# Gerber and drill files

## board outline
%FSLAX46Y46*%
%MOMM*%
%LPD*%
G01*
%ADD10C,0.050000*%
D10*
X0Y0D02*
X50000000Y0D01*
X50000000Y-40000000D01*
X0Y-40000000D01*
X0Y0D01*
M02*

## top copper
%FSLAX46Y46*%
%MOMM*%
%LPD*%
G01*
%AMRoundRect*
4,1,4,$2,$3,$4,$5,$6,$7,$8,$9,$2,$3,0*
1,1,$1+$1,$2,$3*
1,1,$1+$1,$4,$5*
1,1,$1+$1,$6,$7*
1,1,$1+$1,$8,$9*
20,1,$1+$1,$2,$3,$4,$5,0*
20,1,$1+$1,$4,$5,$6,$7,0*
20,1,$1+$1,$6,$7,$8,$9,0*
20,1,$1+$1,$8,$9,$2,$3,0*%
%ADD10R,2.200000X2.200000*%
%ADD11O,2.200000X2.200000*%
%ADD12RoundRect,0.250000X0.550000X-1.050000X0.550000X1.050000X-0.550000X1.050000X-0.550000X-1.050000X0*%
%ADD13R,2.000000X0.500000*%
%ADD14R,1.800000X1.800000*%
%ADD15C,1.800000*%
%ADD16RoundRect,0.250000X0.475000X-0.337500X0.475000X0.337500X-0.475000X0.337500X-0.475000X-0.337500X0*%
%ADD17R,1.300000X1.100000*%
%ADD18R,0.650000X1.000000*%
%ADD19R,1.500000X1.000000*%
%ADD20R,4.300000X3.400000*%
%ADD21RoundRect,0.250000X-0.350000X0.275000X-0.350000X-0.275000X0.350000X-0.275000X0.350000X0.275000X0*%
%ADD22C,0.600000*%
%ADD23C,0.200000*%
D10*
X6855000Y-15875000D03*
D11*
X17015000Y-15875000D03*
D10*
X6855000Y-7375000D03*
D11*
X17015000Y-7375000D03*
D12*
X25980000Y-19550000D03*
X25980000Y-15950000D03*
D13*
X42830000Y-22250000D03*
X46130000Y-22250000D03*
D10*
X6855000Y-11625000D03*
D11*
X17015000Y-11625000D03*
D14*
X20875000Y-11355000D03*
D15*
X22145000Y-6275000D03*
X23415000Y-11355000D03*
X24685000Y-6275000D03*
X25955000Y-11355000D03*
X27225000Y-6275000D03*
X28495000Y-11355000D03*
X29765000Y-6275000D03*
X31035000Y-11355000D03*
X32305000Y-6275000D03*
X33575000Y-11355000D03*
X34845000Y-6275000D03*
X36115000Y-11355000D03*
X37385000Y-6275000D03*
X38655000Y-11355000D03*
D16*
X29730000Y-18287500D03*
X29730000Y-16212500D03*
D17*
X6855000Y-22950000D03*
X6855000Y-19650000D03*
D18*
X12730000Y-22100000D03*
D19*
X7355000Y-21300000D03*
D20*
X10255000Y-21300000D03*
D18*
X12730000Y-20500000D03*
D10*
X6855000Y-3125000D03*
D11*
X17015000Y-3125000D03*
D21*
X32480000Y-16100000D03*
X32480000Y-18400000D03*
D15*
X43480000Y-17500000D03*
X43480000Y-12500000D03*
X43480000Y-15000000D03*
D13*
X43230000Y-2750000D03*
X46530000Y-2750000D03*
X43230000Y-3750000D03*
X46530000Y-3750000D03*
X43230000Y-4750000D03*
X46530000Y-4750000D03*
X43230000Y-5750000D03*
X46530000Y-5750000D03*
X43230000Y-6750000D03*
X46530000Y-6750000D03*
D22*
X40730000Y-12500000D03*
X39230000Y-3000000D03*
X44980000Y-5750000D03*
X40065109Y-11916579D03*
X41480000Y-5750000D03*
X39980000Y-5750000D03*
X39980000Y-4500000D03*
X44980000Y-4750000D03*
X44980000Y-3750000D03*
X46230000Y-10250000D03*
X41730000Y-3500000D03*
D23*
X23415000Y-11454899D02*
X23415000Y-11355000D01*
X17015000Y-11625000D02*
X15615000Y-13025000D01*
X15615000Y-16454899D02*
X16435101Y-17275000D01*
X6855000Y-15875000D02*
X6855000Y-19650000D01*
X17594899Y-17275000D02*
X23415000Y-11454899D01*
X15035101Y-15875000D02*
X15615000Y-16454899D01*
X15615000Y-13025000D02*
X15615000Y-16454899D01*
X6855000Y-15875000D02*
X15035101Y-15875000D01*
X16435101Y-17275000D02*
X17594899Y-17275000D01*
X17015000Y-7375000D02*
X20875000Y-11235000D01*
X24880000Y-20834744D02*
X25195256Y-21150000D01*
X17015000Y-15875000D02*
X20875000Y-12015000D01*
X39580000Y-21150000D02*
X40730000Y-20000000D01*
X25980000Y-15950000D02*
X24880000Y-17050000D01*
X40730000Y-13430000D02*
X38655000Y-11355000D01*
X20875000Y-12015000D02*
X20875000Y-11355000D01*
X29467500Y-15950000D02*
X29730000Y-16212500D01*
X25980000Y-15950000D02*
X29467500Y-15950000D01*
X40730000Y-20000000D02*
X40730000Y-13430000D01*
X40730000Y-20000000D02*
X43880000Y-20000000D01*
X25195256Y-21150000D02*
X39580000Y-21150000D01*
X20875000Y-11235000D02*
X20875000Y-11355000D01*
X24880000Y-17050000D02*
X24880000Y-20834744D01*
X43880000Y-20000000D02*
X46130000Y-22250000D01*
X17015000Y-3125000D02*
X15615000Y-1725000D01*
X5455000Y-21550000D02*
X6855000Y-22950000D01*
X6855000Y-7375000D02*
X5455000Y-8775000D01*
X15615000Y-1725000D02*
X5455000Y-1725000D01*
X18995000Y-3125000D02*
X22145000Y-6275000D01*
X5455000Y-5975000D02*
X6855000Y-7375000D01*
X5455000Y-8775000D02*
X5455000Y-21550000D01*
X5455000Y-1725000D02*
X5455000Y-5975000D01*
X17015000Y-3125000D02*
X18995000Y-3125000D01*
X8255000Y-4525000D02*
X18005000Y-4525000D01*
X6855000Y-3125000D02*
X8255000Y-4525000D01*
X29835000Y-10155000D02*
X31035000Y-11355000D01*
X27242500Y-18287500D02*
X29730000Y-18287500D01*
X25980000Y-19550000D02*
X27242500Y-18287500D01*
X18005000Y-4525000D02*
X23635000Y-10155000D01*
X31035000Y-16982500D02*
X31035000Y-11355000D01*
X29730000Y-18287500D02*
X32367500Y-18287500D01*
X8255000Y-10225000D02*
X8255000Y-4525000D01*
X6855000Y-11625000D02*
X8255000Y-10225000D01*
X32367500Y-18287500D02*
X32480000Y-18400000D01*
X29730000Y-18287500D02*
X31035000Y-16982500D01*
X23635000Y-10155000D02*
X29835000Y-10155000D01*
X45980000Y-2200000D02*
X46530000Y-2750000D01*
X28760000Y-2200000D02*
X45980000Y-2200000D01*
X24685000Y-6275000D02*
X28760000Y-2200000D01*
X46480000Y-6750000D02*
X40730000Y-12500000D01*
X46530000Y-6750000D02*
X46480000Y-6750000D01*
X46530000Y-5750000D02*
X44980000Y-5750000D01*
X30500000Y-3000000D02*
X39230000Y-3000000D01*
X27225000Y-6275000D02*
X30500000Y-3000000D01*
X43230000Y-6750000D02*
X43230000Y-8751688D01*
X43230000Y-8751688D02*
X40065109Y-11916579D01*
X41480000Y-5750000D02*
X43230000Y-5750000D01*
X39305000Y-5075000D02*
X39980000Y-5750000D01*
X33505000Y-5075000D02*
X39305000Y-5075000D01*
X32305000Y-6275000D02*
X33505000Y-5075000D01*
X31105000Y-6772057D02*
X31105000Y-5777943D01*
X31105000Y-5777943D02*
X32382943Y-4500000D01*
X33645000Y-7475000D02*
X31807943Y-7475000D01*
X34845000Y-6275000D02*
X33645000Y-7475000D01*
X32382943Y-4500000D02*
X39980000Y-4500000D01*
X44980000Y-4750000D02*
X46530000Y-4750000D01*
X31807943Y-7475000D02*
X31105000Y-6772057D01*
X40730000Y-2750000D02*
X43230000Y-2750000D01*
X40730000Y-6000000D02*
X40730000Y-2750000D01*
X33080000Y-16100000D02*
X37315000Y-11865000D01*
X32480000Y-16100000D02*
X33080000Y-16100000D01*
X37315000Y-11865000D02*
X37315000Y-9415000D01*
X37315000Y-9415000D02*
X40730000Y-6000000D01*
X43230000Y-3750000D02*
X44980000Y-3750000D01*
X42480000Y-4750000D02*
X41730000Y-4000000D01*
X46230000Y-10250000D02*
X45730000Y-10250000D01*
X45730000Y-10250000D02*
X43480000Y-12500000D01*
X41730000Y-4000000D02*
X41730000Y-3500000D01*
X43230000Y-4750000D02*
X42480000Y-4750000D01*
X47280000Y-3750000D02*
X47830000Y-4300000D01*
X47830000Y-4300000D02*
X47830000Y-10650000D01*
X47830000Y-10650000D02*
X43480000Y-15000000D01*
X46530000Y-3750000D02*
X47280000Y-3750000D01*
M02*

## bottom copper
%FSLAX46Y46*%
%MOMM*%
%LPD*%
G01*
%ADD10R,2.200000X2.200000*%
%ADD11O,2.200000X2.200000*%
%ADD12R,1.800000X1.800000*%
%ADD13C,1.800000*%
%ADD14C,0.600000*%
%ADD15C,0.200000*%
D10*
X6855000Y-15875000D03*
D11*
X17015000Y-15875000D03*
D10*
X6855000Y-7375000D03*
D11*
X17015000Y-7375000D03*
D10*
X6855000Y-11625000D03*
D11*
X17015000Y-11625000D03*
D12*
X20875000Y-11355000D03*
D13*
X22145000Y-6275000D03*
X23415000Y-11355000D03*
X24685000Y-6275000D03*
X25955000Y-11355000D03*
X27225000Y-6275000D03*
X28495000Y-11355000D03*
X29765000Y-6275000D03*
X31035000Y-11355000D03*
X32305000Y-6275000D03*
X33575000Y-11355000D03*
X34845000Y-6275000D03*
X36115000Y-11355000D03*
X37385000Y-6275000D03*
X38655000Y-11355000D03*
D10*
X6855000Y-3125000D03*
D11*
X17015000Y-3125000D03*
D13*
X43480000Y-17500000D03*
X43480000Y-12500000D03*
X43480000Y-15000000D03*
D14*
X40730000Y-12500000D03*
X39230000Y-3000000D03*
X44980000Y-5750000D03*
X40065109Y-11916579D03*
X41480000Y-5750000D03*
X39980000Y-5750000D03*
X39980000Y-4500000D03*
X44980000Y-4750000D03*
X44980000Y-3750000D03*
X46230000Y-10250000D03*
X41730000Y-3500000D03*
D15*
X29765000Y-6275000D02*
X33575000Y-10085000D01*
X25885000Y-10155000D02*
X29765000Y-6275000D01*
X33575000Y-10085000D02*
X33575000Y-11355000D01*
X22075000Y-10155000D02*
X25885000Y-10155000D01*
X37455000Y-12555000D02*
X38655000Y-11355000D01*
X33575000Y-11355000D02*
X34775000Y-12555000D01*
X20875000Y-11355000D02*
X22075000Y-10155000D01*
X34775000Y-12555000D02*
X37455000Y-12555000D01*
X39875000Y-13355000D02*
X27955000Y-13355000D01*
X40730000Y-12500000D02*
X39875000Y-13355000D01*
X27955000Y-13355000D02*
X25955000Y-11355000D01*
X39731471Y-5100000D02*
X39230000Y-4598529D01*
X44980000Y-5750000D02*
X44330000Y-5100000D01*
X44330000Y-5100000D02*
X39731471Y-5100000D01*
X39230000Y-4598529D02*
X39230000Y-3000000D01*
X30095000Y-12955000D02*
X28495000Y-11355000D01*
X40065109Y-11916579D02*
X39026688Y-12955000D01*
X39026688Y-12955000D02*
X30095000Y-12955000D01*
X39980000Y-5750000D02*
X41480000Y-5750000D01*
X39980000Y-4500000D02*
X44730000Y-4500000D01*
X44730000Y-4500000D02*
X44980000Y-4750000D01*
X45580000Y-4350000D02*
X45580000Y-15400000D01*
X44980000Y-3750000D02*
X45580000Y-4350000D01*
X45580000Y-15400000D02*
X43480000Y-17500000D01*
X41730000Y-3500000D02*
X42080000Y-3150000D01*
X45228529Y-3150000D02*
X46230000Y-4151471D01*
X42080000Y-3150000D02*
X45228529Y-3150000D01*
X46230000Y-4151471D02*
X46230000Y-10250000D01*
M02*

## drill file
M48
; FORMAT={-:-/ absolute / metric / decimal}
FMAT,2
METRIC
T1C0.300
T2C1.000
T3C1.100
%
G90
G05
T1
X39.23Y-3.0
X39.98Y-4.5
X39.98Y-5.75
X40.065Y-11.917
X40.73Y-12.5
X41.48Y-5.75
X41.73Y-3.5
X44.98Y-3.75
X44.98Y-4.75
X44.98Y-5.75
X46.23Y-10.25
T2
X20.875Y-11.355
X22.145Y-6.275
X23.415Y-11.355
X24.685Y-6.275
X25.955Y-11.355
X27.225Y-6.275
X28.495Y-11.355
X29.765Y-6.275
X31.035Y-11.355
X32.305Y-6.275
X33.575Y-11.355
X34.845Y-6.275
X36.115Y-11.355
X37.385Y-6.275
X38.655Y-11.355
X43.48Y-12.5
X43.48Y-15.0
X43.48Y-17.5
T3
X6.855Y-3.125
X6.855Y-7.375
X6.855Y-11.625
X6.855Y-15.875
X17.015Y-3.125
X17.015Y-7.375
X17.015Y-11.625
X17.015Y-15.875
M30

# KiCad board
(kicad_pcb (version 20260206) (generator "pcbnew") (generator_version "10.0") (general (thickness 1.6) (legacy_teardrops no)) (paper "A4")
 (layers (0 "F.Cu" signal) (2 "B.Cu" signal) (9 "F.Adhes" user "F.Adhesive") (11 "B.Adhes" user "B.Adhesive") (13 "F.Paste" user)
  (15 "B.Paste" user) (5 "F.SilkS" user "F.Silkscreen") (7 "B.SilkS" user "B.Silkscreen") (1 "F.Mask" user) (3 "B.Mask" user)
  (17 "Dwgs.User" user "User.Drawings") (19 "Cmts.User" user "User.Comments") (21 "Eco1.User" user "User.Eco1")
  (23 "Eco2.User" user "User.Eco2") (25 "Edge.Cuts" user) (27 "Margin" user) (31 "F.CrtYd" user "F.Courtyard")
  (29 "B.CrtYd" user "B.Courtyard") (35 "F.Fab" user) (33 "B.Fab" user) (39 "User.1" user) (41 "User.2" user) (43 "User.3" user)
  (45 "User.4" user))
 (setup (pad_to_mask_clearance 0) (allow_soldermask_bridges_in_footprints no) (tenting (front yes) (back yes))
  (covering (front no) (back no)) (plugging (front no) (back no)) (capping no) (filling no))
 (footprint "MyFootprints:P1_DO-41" (layer "F.Cu") (at 6.855 15.875)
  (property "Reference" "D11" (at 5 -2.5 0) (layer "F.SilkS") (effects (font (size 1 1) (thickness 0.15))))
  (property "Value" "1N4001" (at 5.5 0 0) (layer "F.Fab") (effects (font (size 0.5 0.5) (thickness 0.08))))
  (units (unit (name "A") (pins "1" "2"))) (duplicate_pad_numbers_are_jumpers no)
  (pad "1" thru_hole rect (at 0 0) (size 2.2 2.2) (drill 1.1) (layers "*.Cu" "*.Mask") (remove_unused_layers no) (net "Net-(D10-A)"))
  (pad "2" thru_hole oval (at 10.16 0) (size 2.2 2.2) (drill 1.1) (layers "*.Cu" "*.Mask") (remove_unused_layers no) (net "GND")))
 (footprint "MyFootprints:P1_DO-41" (layer "F.Cu") (at 6.855 7.375)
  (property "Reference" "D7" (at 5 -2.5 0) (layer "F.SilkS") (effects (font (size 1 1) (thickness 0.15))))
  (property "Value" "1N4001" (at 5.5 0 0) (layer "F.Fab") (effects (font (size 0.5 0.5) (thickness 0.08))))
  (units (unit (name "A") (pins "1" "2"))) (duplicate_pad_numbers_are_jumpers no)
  (pad "1" thru_hole rect (at 0 0) (size 2.2 2.2) (drill 1.1) (layers "*.Cu" "*.Mask") (remove_unused_layers no) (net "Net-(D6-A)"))
  (pad "2" thru_hole oval (at 10.16 0) (size 2.2 2.2) (drill 1.1) (layers "*.Cu" "*.Mask") (remove_unused_layers no) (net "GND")))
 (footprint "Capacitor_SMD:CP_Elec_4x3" (layer "F.Cu") (at 25.98 17.75 90)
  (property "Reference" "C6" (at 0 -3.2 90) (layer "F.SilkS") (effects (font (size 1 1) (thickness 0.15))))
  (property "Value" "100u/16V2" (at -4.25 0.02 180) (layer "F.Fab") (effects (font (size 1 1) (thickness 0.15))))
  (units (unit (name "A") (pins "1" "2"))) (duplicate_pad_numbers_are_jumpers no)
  (pad "1" smd roundrect (at -1.8 0 90) (size 2.6 1.6) (layers "F.Cu" "F.Mask" "F.Paste") (roundrect_rratio 0.15625) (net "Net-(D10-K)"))
  (pad "2" smd roundrect (at 1.8 0 90) (size 2.6 1.6) (layers "F.Cu" "F.Mask" "F.Paste") (roundrect_rratio 0.15625) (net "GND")))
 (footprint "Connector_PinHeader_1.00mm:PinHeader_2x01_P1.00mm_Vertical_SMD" (layer "F.Cu") (at 44.48 22.25)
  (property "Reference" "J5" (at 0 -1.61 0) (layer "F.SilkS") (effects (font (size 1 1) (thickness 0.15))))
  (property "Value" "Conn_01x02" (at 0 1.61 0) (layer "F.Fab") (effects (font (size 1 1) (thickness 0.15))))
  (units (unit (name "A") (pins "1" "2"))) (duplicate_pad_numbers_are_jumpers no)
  (pad "1" smd rect (at -1.65 0) (size 2 0.5) (layers "F.Cu" "F.Mask" "F.Paste") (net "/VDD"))
  (pad "2" smd rect (at 1.65 0) (size 2 0.5) (layers "F.Cu" "F.Mask" "F.Paste") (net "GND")))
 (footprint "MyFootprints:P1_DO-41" (layer "F.Cu") (at 6.855 11.625)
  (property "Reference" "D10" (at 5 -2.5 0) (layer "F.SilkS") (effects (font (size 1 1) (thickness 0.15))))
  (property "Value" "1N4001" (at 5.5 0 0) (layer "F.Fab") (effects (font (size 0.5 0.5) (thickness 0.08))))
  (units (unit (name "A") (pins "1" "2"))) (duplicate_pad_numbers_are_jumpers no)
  (pad "1" thru_hole rect (at 0 0) (size 2.2 2.2) (drill 1.1) (layers "*.Cu" "*.Mask") (remove_unused_layers no) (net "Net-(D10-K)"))
  (pad "2" thru_hole oval (at 10.16 0) (size 2.2 2.2) (drill 1.1) (layers "*.Cu" "*.Mask") (remove_unused_layers no) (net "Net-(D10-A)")))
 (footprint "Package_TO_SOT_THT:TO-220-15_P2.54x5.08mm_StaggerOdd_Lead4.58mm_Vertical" (layer "F.Cu") (at 20.875 11.355)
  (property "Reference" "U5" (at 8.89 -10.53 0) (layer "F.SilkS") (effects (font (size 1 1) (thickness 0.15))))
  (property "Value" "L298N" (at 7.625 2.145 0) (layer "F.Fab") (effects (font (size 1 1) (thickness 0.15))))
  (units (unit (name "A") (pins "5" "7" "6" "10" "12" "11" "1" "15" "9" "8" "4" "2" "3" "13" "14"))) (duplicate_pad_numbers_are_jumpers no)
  (pad "1" thru_hole rect (at 0 0) (size 1.8 1.8) (drill 1) (layers "*.Cu" "*.Mask") (remove_unused_layers no) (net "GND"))
  (pad "2" thru_hole circle (at 1.27 -5.08) (size 1.8 1.8) (drill 1) (layers "*.Cu" "*.Mask") (remove_unused_layers no) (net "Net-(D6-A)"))
  (pad "3" thru_hole circle (at 2.54 0) (size 1.8 1.8) (drill 1) (layers "*.Cu" "*.Mask") (remove_unused_layers no) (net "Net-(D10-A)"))
  (pad "4" thru_hole circle (at 3.81 -5.08) (size 1.8 1.8) (drill 1) (layers "*.Cu" "*.Mask") (remove_unused_layers no) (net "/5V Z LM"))
  (pad "5" thru_hole circle (at 5.08 0) (size 1.8 1.8) (drill 1) (layers "*.Cu" "*.Mask") (remove_unused_layers no) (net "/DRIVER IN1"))
  (pad "6" thru_hole circle (at 6.35 -5.08) (size 1.8 1.8) (drill 1) (layers "*.Cu" "*.Mask") (remove_unused_layers no) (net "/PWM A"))
  (pad "7" thru_hole circle (at 7.62 0) (size 1.8 1.8) (drill 1) (layers "*.Cu" "*.Mask") (remove_unused_layers no) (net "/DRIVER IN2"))
  (pad "8" thru_hole circle (at 8.89 -5.08) (size 1.8 1.8) (drill 1) (layers "*.Cu" "*.Mask") (remove_unused_layers no) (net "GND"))
  (pad "9" thru_hole circle (at 10.16 0) (size 1.8 1.8) (drill 1) (layers "*.Cu" "*.Mask") (remove_unused_layers no) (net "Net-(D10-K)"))
  (pad "10" thru_hole circle (at 11.43 -5.08) (size 1.8 1.8) (drill 1) (layers "*.Cu" "*.Mask") (remove_unused_layers no)
   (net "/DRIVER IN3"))
  (pad "11" thru_hole circle (at 12.7 0) (size 1.8 1.8) (drill 1) (layers "*.Cu" "*.Mask") (remove_unused_layers no) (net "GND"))
  (pad "12" thru_hole circle (at 13.97 -5.08) (size 1.8 1.8) (drill 1) (layers "*.Cu" "*.Mask") (remove_unused_layers no)
   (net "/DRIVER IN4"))
  (pad "13" thru_hole circle (at 15.24 0) (size 1.8 1.8) (drill 1) (layers "*.Cu" "*.Mask") (remove_unused_layers no)
   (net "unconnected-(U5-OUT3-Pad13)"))
  (pad "14" thru_hole circle (at 16.51 -5.08) (size 1.8 1.8) (drill 1) (layers "*.Cu" "*.Mask") (remove_unused_layers no)
   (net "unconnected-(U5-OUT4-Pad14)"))
  (pad "15" thru_hole circle (at 17.78 0) (size 1.8 1.8) (drill 1) (layers "*.Cu" "*.Mask") (remove_unused_layers no) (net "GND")))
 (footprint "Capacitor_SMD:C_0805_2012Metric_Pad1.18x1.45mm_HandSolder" (layer "F.Cu") (at 29.73 17.25 90)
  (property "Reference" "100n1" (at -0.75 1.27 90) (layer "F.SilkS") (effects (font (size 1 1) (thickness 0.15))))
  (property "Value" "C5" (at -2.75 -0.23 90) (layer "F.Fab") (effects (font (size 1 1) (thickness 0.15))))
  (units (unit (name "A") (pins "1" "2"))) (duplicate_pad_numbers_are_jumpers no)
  (pad "1" smd roundrect (at -1.0375 0 90) (size 1.175 1.45) (layers "F.Cu" "F.Mask" "F.Paste") (roundrect_rratio 0.212766)
   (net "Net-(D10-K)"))
  (pad "2" smd roundrect (at 1.0375 0 90) (size 1.175 1.45) (layers "F.Cu" "F.Mask" "F.Paste") (roundrect_rratio 0.212766) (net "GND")))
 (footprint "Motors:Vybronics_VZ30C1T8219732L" (layer "F.Cu") (at 11.205 21.3 90)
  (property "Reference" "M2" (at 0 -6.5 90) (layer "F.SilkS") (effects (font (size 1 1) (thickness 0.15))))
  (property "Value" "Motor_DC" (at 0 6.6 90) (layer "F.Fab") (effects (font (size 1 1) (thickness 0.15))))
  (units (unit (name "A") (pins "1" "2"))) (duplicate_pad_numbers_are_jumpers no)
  (pad "" smd rect (at -0.85 -2.315) (size 1.07 1.4) (layers "F.Paste"))
  (pad "" smd rect (at -0.85 -0.905) (size 1.07 1.4) (layers "F.Paste"))
  (pad "" smd rect (at -0.85 0.505) (size 1.07 1.4) (layers "F.Paste"))
  (pad "" smd rect (at 0.85 -2.315) (size 1.07 1.4) (layers "F.Paste"))
  (pad "" smd rect (at 0.85 -0.905) (size 1.07 1.4) (layers "F.Paste"))
  (pad "" smd rect (at 0.85 0.505) (size 1.07 1.4) (layers "F.Paste"))
  (pad "1" smd rect (at -1.65 -4.35) (size 1.3 1.1) (layers "F.Cu" "F.Mask" "F.Paste") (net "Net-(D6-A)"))
  (pad "2" smd rect (at 1.65 -4.35) (size 1.3 1.1) (layers "F.Cu" "F.Mask" "F.Paste") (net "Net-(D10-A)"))
  (pad "SH" smd rect (at -0.8 1.525 90) (size 1 0.65) (layers "F.Cu" "F.Mask" "F.Paste"))
  (pad "SH" smd rect (at 0 -3.85) (size 1.5 1) (layers "F.Cu" "F.Mask" "F.Paste"))
  (pad "SH" smd rect (at 0 -0.95) (size 4.3 3.4) (layers "F.Cu" "F.Mask"))
  (pad "SH" smd rect (at 0.8 1.525 90) (size 1 0.65) (layers "F.Cu" "F.Mask" "F.Paste")))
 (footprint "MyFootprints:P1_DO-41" (layer "F.Cu") (at 6.855 3.125)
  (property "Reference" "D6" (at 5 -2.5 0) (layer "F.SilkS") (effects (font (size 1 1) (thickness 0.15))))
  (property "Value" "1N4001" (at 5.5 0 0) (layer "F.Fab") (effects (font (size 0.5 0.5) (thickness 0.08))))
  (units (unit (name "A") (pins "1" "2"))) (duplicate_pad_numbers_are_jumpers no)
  (pad "1" thru_hole rect (at 0 0) (size 2.2 2.2) (drill 1.1) (layers "*.Cu" "*.Mask") (remove_unused_layers no) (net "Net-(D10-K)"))
  (pad "2" thru_hole oval (at 10.16 0) (size 2.2 2.2) (drill 1.1) (layers "*.Cu" "*.Mask") (remove_unused_layers no) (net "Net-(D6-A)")))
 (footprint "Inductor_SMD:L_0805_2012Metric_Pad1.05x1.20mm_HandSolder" (layer "F.Cu") (at 32.48 17.25 -90)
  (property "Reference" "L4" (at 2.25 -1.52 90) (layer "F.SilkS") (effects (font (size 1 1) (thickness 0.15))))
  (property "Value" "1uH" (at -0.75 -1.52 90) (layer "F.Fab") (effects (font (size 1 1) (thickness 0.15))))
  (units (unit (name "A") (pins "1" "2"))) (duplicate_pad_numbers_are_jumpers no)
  (pad "1" smd roundrect (at -1.15 0 270) (size 1.05 1.2) (layers "F.Cu" "F.Mask" "F.Paste") (roundrect_rratio 0.238095)
   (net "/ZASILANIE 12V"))
  (pad "2" smd roundrect (at 1.15 0 270) (size 1.05 1.2) (layers "F.Cu" "F.Mask" "F.Paste") (roundrect_rratio 0.238095) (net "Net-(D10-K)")))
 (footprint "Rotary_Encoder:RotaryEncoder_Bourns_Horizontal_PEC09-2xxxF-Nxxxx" (layer "F.Cu") (at 43.48 17.5)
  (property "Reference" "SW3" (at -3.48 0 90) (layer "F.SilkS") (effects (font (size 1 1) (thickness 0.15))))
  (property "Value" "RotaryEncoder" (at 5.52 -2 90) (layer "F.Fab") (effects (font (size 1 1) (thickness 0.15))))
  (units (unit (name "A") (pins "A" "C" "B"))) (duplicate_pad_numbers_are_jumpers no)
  (pad "A" thru_hole circle (at 0 0) (size 1.8 1.8) (drill 1) (layers "*.Cu" "*.Mask") (remove_unused_layers no) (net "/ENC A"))
  (pad "B" thru_hole circle (at 0 -5) (size 1.8 1.8) (drill 1) (layers "*.Cu" "*.Mask") (remove_unused_layers no) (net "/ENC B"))
  (pad "C" thru_hole circle (at 0 -2.5) (size 1.8 1.8) (drill 1) (layers "*.Cu" "*.Mask") (remove_unused_layers no) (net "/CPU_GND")))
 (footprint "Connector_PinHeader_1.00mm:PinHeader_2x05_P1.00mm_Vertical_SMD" (layer "F.Cu") (at 44.88 4.75)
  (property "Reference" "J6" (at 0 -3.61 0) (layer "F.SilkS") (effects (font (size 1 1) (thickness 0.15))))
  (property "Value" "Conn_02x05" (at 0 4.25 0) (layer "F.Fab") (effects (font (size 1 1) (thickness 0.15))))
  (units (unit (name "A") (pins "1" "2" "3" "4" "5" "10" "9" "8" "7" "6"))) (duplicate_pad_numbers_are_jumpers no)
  (pad "1" smd rect (at -1.65 -2) (size 2 0.5) (layers "F.Cu" "F.Mask" "F.Paste") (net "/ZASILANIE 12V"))
  (pad "2" smd rect (at 1.65 -2) (size 2 0.5) (layers "F.Cu" "F.Mask" "F.Paste") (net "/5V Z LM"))
  (pad "3" smd rect (at -1.65 -1) (size 2 0.5) (layers "F.Cu" "F.Mask" "F.Paste") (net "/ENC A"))
  (pad "4" smd rect (at 1.65 -1) (size 2 0.5) (layers "F.Cu" "F.Mask" "F.Paste") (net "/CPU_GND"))
  (pad "5" smd rect (at -1.65 0) (size 2 0.5) (layers "F.Cu" "F.Mask" "F.Paste") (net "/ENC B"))
  (pad "6" smd rect (at 1.65 0) (size 2 0.5) (layers "F.Cu" "F.Mask" "F.Paste") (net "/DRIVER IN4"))
  (pad "7" smd rect (at -1.65 1) (size 2 0.5) (layers "F.Cu" "F.Mask" "F.Paste") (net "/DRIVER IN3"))
  (pad "8" smd rect (at 1.65 1) (size 2 0.5) (layers "F.Cu" "F.Mask" "F.Paste") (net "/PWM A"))
  (pad "9" smd rect (at -1.65 2) (size 2 0.5) (layers "F.Cu" "F.Mask" "F.Paste") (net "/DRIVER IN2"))
  (pad "10" smd rect (at 1.65 2) (size 2 0.5) (layers "F.Cu" "F.Mask" "F.Paste") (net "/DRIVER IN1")))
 (gr_rect (start 0 0) (end 50 40) (stroke (width 0.05) (type solid)) (fill no) (layer "Edge.Cuts"))
 (segment (start 23.415 11.454899) (end 23.415 11.355) (width 0.2) (layer "F.Cu") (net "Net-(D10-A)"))
 (segment (start 17.015 11.625) (end 15.615 13.025) (width 0.2) (layer "F.Cu") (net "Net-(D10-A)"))
 (segment (start 15.615 16.454899) (end 16.435101 17.275) (width 0.2) (layer "F.Cu") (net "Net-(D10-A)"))
 (segment (start 6.855 15.875) (end 6.855 19.65) (width 0.2) (layer "F.Cu") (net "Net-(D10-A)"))
 (segment (start 17.594899 17.275) (end 23.415 11.454899) (width 0.2) (layer "F.Cu") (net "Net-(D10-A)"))
 (segment (start 15.035101 15.875) (end 15.615 16.454899) (width 0.2) (layer "F.Cu") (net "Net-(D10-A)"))
 (segment (start 15.615 13.025) (end 15.615 16.454899) (width 0.2) (layer "F.Cu") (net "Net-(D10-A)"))
 (segment (start 6.855 15.875) (end 15.035101 15.875) (width 0.2) (layer "F.Cu") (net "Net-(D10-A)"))
 (segment (start 16.435101 17.275) (end 17.594899 17.275) (width 0.2) (layer "F.Cu") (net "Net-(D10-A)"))
 (segment (start 17.015 7.375) (end 20.875 11.235) (width 0.2) (layer "F.Cu") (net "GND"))
 (segment (start 24.88 20.834744) (end 25.195256 21.15) (width 0.2) (layer "F.Cu") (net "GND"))
 (segment (start 17.015 15.875) (end 20.875 12.015) (width 0.2) (layer "F.Cu") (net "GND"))
 (segment (start 39.58 21.15) (end 40.73 20) (width 0.2) (layer "F.Cu") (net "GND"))
 (segment (start 25.98 15.95) (end 24.88 17.05) (width 0.2) (layer "F.Cu") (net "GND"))
 (segment (start 40.73 13.43) (end 38.655 11.355) (width 0.2) (layer "F.Cu") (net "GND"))
 (segment (start 20.875 12.015) (end 20.875 11.355) (width 0.2) (layer "F.Cu") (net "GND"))
 (segment (start 29.4675 15.95) (end 29.73 16.2125) (width 0.2) (layer "F.Cu") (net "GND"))
 (segment (start 25.98 15.95) (end 29.4675 15.95) (width 0.2) (layer "F.Cu") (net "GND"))
 (segment (start 40.73 20) (end 40.73 13.43) (width 0.2) (layer "F.Cu") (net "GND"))
 (segment (start 40.73 20) (end 43.88 20) (width 0.2) (layer "F.Cu") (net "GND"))
 (segment (start 25.195256 21.15) (end 39.58 21.15) (width 0.2) (layer "F.Cu") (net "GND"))
 (segment (start 20.875 11.235) (end 20.875 11.355) (width 0.2) (layer "F.Cu") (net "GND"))
 (segment (start 24.88 17.05) (end 24.88 20.834744) (width 0.2) (layer "F.Cu") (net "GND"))
 (segment (start 43.88 20) (end 46.13 22.25) (width 0.2) (layer "F.Cu") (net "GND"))
 (segment (start 29.765 6.275) (end 33.575 10.085) (width 0.2) (layer "B.Cu") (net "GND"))
 (segment (start 25.885 10.155) (end 29.765 6.275) (width 0.2) (layer "B.Cu") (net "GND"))
 (segment (start 33.575 10.085) (end 33.575 11.355) (width 0.2) (layer "B.Cu") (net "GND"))
 (segment (start 22.075 10.155) (end 25.885 10.155) (width 0.2) (layer "B.Cu") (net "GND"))
 (segment (start 37.455 12.555) (end 38.655 11.355) (width 0.2) (layer "B.Cu") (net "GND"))
 (segment (start 33.575 11.355) (end 34.775 12.555) (width 0.2) (layer "B.Cu") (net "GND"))
 (segment (start 20.875 11.355) (end 22.075 10.155) (width 0.2) (layer "B.Cu") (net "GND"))
 (segment (start 34.775 12.555) (end 37.455 12.555) (width 0.2) (layer "B.Cu") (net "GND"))
 (segment (start 17.015 3.125) (end 15.615 1.725) (width 0.2) (layer "F.Cu") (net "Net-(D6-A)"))
 (segment (start 5.455 21.55) (end 6.855 22.95) (width 0.2) (layer "F.Cu") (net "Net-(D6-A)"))
 (segment (start 6.855 7.375) (end 5.455 8.775) (width 0.2) (layer "F.Cu") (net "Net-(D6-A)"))
 (segment (start 15.615 1.725) (end 5.455 1.725) (width 0.2) (layer "F.Cu") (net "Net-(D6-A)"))
 (segment (start 18.995 3.125) (end 22.145 6.275) (width 0.2) (layer "F.Cu") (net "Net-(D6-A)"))
 (segment (start 5.455 5.975) (end 6.855 7.375) (width 0.2) (layer "F.Cu") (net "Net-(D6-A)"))
 (segment (start 5.455 8.775) (end 5.455 21.55) (width 0.2) (layer "F.Cu") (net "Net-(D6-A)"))
 (segment (start 5.455 1.725) (end 5.455 5.975) (width 0.2) (layer "F.Cu") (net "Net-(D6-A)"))
 (segment (start 17.015 3.125) (end 18.995 3.125) (width 0.2) (layer "F.Cu") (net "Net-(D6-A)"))
 (segment (start 8.255 4.525) (end 18.005 4.525) (width 0.2) (layer "F.Cu") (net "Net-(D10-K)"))
 (segment (start 6.855 3.125) (end 8.255 4.525) (width 0.2) (layer "F.Cu") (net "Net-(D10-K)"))
 (segment (start 29.835 10.155) (end 31.035 11.355) (width 0.2) (layer "F.Cu") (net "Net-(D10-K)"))
 (segment (start 27.2425 18.2875) (end 29.73 18.2875) (width 0.2) (layer "F.Cu") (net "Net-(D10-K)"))
 (segment (start 25.98 19.55) (end 27.2425 18.2875) (width 0.2) (layer "F.Cu") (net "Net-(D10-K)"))
 (segment (start 18.005 4.525) (end 23.635 10.155) (width 0.2) (layer "F.Cu") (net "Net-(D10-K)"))
 (segment (start 31.035 16.9825) (end 31.035 11.355) (width 0.2) (layer "F.Cu") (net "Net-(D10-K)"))
 (segment (start 29.73 18.2875) (end 32.3675 18.2875) (width 0.2) (layer "F.Cu") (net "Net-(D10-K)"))
 (segment (start 8.255 10.225) (end 8.255 4.525) (width 0.2) (layer "F.Cu") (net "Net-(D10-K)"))
 (segment (start 6.855 11.625) (end 8.255 10.225) (width 0.2) (layer "F.Cu") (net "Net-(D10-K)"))
 (segment (start 32.3675 18.2875) (end 32.48 18.4) (width 0.2) (layer "F.Cu") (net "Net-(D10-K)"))
 (segment (start 29.73 18.2875) (end 31.035 16.9825) (width 0.2) (layer "F.Cu") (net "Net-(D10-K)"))
 (segment (start 23.635 10.155) (end 29.835 10.155) (width 0.2) (layer "F.Cu") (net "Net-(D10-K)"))
 (segment (start 45.98 2.2) (end 46.53 2.75) (width 0.2) (layer "F.Cu") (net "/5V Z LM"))
 (segment (start 28.76 2.2) (end 45.98 2.2) (width 0.2) (layer "F.Cu") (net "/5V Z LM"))
 (segment (start 24.685 6.275) (end 28.76 2.2) (width 0.2) (layer "F.Cu") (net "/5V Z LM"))
 (segment (start 46.48 6.75) (end 40.73 12.5) (width 0.2) (layer "F.Cu") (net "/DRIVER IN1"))
 (segment (start 46.53 6.75) (end 46.48 6.75) (width 0.2) (layer "F.Cu") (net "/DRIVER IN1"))
 (via (at 40.73 12.5) (size 0.6) (drill 0.3) (layers "F.Cu" "B.Cu") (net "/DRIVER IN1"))
 (segment (start 39.875 13.355) (end 27.955 13.355) (width 0.2) (layer "B.Cu") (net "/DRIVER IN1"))
 (segment (start 40.73 12.5) (end 39.875 13.355) (width 0.2) (layer "B.Cu") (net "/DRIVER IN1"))
 (segment (start 27.955 13.355) (end 25.955 11.355) (width 0.2) (layer "B.Cu") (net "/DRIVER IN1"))
 (segment (start 46.53 5.75) (end 44.98 5.75) (width 0.2) (layer "F.Cu") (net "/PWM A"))
 (segment (start 30.5 3) (end 39.23 3) (width 0.2) (layer "F.Cu") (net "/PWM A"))
 (segment (start 27.225 6.275) (end 30.5 3) (width 0.2) (layer "F.Cu") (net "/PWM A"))
 (via (at 39.23 3) (size 0.6) (drill 0.3) (layers "F.Cu" "B.Cu") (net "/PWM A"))
 (via (at 44.98 5.75) (size 0.6) (drill 0.3) (layers "F.Cu" "B.Cu") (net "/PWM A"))
 (segment (start 39.731471 5.1) (end 39.23 4.598529) (width 0.2) (layer "B.Cu") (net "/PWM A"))
 (segment (start 44.98 5.75) (end 44.33 5.1) (width 0.2) (layer "B.Cu") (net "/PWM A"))
 (segment (start 44.33 5.1) (end 39.731471 5.1) (width 0.2) (layer "B.Cu") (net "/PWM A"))
 (segment (start 39.23 4.598529) (end 39.23 3) (width 0.2) (layer "B.Cu") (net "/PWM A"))
 (segment (start 43.23 6.75) (end 43.23 8.751688) (width 0.2) (layer "F.Cu") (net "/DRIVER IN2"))
 (segment (start 43.23 8.751688) (end 40.065109 11.916579) (width 0.2) (layer "F.Cu") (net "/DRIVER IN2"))
 (via (at 40.065109 11.916579) (size 0.6) (drill 0.3) (layers "F.Cu" "B.Cu") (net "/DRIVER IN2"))
 (segment (start 30.095 12.955) (end 28.495 11.355) (width 0.2) (layer "B.Cu") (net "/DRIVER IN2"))
 (segment (start 40.065109 11.916579) (end 39.026688 12.955) (width 0.2) (layer "B.Cu") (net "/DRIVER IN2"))
 (segment (start 39.026688 12.955) (end 30.095 12.955) (width 0.2) (layer "B.Cu") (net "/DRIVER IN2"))
 (segment (start 41.48 5.75) (end 43.23 5.75) (width 0.2) (layer "F.Cu") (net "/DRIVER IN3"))
 (segment (start 39.305 5.075) (end 39.98 5.75) (width 0.2) (layer "F.Cu") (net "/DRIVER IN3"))
 (segment (start 33.505 5.075) (end 39.305 5.075) (width 0.2) (layer "F.Cu") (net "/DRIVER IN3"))
 (segment (start 32.305 6.275) (end 33.505 5.075) (width 0.2) (layer "F.Cu") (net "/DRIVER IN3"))
 (via (at 41.48 5.75) (size 0.6) (drill 0.3) (layers "F.Cu" "B.Cu") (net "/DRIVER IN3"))
 (via (at 39.98 5.75) (size 0.6) (drill 0.3) (layers "F.Cu" "B.Cu") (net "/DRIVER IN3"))
 (segment (start 39.98 5.75) (end 41.48 5.75) (width 0.2) (layer "B.Cu") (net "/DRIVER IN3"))
 (segment (start 31.105 6.772057) (end 31.105 5.777943) (width 0.2) (layer "F.Cu") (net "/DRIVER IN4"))
 (segment (start 31.105 5.777943) (end 32.382943 4.5) (width 0.2) (layer "F.Cu") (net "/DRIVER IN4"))
 (segment (start 33.645 7.475) (end 31.807943 7.475) (width 0.2) (layer "F.Cu") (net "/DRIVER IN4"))
 (segment (start 34.845 6.275) (end 33.645 7.475) (width 0.2) (layer "F.Cu") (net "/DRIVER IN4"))
 (segment (start 32.382943 4.5) (end 39.98 4.5) (width 0.2) (layer "F.Cu") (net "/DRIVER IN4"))
 (segment (start 44.98 4.75) (end 46.53 4.75) (width 0.2) (layer "F.Cu") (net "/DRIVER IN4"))
 (segment (start 31.807943 7.475) (end 31.105 6.772057) (width 0.2) (layer "F.Cu") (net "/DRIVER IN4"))
 (via (at 39.98 4.5) (size 0.6) (drill 0.3) (layers "F.Cu" "B.Cu") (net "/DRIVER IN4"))
 (via (at 44.98 4.75) (size 0.6) (drill 0.3) (layers "F.Cu" "B.Cu") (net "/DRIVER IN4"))
 (segment (start 39.98 4.5) (end 44.73 4.5) (width 0.2) (layer "B.Cu") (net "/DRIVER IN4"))
 (segment (start 44.73 4.5) (end 44.98 4.75) (width 0.2) (layer "B.Cu") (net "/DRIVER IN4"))
 (segment (start 40.73 2.75) (end 43.23 2.75) (width 0.2) (layer "F.Cu") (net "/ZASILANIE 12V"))
 (segment (start 40.73 6) (end 40.73 2.75) (width 0.2) (layer "F.Cu") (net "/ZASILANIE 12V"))
 (segment (start 33.08 16.1) (end 37.315 11.865) (width 0.2) (layer "F.Cu") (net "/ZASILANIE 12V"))
 (segment (start 32.48 16.1) (end 33.08 16.1) (width 0.2) (layer "F.Cu") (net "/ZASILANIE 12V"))
 (segment (start 37.315 11.865) (end 37.315 9.415) (width 0.2) (layer "F.Cu") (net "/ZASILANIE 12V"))
 (segment (start 37.315 9.415) (end 40.73 6) (width 0.2) (layer "F.Cu") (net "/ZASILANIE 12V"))
 (segment (start 43.23 3.75) (end 44.98 3.75) (width 0.2) (layer "F.Cu") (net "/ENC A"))
 (via (at 44.98 3.75) (size 0.6) (drill 0.3) (layers "F.Cu" "B.Cu") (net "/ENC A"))
 (segment (start 45.58 4.35) (end 45.58 15.4) (width 0.2) (layer "B.Cu") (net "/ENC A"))
 (segment (start 44.98 3.75) (end 45.58 4.35) (width 0.2) (layer "B.Cu") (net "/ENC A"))
 (segment (start 45.58 15.4) (end 43.48 17.5) (width 0.2) (layer "B.Cu") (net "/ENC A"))
 (segment (start 42.48 4.75) (end 41.73 4) (width 0.2) (layer "F.Cu") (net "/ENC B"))
 (segment (start 46.23 10.25) (end 45.73 10.25) (width 0.2) (layer "F.Cu") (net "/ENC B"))
 (segment (start 45.73 10.25) (end 43.48 12.5) (width 0.2) (layer "F.Cu") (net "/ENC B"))
 (segment (start 41.73 4) (end 41.73 3.5) (width 0.2) (layer "F.Cu") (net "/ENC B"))
 (segment (start 43.23 4.75) (end 42.48 4.75) (width 0.2) (layer "F.Cu") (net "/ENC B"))
 (via (at 46.23 10.25) (size 0.6) (drill 0.3) (layers "F.Cu" "B.Cu") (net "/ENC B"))
 (via (at 41.73 3.5) (size 0.6) (drill 0.3) (layers "F.Cu" "B.Cu") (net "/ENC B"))
 (segment (start 41.73 3.5) (end 42.08 3.15) (width 0.2) (layer "B.Cu") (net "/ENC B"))
 (segment (start 45.228529 3.15) (end 46.23 4.151471) (width 0.2) (layer "B.Cu") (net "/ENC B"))
 (segment (start 42.08 3.15) (end 45.228529 3.15) (width 0.2) (layer "B.Cu") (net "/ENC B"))
 (segment (start 46.23 4.151471) (end 46.23 10.25) (width 0.2) (layer "B.Cu") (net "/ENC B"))
 (segment (start 47.28 3.75) (end 47.83 4.3) (width 0.2) (layer "F.Cu") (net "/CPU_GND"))
 (segment (start 47.83 4.3) (end 47.83 10.65) (width 0.2) (layer "F.Cu") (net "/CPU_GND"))
 (segment (start 47.83 10.65) (end 43.48 15) (width 0.2) (layer "F.Cu") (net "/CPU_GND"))
 (segment (start 46.53 3.75) (end 47.28 3.75) (width 0.2) (layer "F.Cu") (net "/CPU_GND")))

